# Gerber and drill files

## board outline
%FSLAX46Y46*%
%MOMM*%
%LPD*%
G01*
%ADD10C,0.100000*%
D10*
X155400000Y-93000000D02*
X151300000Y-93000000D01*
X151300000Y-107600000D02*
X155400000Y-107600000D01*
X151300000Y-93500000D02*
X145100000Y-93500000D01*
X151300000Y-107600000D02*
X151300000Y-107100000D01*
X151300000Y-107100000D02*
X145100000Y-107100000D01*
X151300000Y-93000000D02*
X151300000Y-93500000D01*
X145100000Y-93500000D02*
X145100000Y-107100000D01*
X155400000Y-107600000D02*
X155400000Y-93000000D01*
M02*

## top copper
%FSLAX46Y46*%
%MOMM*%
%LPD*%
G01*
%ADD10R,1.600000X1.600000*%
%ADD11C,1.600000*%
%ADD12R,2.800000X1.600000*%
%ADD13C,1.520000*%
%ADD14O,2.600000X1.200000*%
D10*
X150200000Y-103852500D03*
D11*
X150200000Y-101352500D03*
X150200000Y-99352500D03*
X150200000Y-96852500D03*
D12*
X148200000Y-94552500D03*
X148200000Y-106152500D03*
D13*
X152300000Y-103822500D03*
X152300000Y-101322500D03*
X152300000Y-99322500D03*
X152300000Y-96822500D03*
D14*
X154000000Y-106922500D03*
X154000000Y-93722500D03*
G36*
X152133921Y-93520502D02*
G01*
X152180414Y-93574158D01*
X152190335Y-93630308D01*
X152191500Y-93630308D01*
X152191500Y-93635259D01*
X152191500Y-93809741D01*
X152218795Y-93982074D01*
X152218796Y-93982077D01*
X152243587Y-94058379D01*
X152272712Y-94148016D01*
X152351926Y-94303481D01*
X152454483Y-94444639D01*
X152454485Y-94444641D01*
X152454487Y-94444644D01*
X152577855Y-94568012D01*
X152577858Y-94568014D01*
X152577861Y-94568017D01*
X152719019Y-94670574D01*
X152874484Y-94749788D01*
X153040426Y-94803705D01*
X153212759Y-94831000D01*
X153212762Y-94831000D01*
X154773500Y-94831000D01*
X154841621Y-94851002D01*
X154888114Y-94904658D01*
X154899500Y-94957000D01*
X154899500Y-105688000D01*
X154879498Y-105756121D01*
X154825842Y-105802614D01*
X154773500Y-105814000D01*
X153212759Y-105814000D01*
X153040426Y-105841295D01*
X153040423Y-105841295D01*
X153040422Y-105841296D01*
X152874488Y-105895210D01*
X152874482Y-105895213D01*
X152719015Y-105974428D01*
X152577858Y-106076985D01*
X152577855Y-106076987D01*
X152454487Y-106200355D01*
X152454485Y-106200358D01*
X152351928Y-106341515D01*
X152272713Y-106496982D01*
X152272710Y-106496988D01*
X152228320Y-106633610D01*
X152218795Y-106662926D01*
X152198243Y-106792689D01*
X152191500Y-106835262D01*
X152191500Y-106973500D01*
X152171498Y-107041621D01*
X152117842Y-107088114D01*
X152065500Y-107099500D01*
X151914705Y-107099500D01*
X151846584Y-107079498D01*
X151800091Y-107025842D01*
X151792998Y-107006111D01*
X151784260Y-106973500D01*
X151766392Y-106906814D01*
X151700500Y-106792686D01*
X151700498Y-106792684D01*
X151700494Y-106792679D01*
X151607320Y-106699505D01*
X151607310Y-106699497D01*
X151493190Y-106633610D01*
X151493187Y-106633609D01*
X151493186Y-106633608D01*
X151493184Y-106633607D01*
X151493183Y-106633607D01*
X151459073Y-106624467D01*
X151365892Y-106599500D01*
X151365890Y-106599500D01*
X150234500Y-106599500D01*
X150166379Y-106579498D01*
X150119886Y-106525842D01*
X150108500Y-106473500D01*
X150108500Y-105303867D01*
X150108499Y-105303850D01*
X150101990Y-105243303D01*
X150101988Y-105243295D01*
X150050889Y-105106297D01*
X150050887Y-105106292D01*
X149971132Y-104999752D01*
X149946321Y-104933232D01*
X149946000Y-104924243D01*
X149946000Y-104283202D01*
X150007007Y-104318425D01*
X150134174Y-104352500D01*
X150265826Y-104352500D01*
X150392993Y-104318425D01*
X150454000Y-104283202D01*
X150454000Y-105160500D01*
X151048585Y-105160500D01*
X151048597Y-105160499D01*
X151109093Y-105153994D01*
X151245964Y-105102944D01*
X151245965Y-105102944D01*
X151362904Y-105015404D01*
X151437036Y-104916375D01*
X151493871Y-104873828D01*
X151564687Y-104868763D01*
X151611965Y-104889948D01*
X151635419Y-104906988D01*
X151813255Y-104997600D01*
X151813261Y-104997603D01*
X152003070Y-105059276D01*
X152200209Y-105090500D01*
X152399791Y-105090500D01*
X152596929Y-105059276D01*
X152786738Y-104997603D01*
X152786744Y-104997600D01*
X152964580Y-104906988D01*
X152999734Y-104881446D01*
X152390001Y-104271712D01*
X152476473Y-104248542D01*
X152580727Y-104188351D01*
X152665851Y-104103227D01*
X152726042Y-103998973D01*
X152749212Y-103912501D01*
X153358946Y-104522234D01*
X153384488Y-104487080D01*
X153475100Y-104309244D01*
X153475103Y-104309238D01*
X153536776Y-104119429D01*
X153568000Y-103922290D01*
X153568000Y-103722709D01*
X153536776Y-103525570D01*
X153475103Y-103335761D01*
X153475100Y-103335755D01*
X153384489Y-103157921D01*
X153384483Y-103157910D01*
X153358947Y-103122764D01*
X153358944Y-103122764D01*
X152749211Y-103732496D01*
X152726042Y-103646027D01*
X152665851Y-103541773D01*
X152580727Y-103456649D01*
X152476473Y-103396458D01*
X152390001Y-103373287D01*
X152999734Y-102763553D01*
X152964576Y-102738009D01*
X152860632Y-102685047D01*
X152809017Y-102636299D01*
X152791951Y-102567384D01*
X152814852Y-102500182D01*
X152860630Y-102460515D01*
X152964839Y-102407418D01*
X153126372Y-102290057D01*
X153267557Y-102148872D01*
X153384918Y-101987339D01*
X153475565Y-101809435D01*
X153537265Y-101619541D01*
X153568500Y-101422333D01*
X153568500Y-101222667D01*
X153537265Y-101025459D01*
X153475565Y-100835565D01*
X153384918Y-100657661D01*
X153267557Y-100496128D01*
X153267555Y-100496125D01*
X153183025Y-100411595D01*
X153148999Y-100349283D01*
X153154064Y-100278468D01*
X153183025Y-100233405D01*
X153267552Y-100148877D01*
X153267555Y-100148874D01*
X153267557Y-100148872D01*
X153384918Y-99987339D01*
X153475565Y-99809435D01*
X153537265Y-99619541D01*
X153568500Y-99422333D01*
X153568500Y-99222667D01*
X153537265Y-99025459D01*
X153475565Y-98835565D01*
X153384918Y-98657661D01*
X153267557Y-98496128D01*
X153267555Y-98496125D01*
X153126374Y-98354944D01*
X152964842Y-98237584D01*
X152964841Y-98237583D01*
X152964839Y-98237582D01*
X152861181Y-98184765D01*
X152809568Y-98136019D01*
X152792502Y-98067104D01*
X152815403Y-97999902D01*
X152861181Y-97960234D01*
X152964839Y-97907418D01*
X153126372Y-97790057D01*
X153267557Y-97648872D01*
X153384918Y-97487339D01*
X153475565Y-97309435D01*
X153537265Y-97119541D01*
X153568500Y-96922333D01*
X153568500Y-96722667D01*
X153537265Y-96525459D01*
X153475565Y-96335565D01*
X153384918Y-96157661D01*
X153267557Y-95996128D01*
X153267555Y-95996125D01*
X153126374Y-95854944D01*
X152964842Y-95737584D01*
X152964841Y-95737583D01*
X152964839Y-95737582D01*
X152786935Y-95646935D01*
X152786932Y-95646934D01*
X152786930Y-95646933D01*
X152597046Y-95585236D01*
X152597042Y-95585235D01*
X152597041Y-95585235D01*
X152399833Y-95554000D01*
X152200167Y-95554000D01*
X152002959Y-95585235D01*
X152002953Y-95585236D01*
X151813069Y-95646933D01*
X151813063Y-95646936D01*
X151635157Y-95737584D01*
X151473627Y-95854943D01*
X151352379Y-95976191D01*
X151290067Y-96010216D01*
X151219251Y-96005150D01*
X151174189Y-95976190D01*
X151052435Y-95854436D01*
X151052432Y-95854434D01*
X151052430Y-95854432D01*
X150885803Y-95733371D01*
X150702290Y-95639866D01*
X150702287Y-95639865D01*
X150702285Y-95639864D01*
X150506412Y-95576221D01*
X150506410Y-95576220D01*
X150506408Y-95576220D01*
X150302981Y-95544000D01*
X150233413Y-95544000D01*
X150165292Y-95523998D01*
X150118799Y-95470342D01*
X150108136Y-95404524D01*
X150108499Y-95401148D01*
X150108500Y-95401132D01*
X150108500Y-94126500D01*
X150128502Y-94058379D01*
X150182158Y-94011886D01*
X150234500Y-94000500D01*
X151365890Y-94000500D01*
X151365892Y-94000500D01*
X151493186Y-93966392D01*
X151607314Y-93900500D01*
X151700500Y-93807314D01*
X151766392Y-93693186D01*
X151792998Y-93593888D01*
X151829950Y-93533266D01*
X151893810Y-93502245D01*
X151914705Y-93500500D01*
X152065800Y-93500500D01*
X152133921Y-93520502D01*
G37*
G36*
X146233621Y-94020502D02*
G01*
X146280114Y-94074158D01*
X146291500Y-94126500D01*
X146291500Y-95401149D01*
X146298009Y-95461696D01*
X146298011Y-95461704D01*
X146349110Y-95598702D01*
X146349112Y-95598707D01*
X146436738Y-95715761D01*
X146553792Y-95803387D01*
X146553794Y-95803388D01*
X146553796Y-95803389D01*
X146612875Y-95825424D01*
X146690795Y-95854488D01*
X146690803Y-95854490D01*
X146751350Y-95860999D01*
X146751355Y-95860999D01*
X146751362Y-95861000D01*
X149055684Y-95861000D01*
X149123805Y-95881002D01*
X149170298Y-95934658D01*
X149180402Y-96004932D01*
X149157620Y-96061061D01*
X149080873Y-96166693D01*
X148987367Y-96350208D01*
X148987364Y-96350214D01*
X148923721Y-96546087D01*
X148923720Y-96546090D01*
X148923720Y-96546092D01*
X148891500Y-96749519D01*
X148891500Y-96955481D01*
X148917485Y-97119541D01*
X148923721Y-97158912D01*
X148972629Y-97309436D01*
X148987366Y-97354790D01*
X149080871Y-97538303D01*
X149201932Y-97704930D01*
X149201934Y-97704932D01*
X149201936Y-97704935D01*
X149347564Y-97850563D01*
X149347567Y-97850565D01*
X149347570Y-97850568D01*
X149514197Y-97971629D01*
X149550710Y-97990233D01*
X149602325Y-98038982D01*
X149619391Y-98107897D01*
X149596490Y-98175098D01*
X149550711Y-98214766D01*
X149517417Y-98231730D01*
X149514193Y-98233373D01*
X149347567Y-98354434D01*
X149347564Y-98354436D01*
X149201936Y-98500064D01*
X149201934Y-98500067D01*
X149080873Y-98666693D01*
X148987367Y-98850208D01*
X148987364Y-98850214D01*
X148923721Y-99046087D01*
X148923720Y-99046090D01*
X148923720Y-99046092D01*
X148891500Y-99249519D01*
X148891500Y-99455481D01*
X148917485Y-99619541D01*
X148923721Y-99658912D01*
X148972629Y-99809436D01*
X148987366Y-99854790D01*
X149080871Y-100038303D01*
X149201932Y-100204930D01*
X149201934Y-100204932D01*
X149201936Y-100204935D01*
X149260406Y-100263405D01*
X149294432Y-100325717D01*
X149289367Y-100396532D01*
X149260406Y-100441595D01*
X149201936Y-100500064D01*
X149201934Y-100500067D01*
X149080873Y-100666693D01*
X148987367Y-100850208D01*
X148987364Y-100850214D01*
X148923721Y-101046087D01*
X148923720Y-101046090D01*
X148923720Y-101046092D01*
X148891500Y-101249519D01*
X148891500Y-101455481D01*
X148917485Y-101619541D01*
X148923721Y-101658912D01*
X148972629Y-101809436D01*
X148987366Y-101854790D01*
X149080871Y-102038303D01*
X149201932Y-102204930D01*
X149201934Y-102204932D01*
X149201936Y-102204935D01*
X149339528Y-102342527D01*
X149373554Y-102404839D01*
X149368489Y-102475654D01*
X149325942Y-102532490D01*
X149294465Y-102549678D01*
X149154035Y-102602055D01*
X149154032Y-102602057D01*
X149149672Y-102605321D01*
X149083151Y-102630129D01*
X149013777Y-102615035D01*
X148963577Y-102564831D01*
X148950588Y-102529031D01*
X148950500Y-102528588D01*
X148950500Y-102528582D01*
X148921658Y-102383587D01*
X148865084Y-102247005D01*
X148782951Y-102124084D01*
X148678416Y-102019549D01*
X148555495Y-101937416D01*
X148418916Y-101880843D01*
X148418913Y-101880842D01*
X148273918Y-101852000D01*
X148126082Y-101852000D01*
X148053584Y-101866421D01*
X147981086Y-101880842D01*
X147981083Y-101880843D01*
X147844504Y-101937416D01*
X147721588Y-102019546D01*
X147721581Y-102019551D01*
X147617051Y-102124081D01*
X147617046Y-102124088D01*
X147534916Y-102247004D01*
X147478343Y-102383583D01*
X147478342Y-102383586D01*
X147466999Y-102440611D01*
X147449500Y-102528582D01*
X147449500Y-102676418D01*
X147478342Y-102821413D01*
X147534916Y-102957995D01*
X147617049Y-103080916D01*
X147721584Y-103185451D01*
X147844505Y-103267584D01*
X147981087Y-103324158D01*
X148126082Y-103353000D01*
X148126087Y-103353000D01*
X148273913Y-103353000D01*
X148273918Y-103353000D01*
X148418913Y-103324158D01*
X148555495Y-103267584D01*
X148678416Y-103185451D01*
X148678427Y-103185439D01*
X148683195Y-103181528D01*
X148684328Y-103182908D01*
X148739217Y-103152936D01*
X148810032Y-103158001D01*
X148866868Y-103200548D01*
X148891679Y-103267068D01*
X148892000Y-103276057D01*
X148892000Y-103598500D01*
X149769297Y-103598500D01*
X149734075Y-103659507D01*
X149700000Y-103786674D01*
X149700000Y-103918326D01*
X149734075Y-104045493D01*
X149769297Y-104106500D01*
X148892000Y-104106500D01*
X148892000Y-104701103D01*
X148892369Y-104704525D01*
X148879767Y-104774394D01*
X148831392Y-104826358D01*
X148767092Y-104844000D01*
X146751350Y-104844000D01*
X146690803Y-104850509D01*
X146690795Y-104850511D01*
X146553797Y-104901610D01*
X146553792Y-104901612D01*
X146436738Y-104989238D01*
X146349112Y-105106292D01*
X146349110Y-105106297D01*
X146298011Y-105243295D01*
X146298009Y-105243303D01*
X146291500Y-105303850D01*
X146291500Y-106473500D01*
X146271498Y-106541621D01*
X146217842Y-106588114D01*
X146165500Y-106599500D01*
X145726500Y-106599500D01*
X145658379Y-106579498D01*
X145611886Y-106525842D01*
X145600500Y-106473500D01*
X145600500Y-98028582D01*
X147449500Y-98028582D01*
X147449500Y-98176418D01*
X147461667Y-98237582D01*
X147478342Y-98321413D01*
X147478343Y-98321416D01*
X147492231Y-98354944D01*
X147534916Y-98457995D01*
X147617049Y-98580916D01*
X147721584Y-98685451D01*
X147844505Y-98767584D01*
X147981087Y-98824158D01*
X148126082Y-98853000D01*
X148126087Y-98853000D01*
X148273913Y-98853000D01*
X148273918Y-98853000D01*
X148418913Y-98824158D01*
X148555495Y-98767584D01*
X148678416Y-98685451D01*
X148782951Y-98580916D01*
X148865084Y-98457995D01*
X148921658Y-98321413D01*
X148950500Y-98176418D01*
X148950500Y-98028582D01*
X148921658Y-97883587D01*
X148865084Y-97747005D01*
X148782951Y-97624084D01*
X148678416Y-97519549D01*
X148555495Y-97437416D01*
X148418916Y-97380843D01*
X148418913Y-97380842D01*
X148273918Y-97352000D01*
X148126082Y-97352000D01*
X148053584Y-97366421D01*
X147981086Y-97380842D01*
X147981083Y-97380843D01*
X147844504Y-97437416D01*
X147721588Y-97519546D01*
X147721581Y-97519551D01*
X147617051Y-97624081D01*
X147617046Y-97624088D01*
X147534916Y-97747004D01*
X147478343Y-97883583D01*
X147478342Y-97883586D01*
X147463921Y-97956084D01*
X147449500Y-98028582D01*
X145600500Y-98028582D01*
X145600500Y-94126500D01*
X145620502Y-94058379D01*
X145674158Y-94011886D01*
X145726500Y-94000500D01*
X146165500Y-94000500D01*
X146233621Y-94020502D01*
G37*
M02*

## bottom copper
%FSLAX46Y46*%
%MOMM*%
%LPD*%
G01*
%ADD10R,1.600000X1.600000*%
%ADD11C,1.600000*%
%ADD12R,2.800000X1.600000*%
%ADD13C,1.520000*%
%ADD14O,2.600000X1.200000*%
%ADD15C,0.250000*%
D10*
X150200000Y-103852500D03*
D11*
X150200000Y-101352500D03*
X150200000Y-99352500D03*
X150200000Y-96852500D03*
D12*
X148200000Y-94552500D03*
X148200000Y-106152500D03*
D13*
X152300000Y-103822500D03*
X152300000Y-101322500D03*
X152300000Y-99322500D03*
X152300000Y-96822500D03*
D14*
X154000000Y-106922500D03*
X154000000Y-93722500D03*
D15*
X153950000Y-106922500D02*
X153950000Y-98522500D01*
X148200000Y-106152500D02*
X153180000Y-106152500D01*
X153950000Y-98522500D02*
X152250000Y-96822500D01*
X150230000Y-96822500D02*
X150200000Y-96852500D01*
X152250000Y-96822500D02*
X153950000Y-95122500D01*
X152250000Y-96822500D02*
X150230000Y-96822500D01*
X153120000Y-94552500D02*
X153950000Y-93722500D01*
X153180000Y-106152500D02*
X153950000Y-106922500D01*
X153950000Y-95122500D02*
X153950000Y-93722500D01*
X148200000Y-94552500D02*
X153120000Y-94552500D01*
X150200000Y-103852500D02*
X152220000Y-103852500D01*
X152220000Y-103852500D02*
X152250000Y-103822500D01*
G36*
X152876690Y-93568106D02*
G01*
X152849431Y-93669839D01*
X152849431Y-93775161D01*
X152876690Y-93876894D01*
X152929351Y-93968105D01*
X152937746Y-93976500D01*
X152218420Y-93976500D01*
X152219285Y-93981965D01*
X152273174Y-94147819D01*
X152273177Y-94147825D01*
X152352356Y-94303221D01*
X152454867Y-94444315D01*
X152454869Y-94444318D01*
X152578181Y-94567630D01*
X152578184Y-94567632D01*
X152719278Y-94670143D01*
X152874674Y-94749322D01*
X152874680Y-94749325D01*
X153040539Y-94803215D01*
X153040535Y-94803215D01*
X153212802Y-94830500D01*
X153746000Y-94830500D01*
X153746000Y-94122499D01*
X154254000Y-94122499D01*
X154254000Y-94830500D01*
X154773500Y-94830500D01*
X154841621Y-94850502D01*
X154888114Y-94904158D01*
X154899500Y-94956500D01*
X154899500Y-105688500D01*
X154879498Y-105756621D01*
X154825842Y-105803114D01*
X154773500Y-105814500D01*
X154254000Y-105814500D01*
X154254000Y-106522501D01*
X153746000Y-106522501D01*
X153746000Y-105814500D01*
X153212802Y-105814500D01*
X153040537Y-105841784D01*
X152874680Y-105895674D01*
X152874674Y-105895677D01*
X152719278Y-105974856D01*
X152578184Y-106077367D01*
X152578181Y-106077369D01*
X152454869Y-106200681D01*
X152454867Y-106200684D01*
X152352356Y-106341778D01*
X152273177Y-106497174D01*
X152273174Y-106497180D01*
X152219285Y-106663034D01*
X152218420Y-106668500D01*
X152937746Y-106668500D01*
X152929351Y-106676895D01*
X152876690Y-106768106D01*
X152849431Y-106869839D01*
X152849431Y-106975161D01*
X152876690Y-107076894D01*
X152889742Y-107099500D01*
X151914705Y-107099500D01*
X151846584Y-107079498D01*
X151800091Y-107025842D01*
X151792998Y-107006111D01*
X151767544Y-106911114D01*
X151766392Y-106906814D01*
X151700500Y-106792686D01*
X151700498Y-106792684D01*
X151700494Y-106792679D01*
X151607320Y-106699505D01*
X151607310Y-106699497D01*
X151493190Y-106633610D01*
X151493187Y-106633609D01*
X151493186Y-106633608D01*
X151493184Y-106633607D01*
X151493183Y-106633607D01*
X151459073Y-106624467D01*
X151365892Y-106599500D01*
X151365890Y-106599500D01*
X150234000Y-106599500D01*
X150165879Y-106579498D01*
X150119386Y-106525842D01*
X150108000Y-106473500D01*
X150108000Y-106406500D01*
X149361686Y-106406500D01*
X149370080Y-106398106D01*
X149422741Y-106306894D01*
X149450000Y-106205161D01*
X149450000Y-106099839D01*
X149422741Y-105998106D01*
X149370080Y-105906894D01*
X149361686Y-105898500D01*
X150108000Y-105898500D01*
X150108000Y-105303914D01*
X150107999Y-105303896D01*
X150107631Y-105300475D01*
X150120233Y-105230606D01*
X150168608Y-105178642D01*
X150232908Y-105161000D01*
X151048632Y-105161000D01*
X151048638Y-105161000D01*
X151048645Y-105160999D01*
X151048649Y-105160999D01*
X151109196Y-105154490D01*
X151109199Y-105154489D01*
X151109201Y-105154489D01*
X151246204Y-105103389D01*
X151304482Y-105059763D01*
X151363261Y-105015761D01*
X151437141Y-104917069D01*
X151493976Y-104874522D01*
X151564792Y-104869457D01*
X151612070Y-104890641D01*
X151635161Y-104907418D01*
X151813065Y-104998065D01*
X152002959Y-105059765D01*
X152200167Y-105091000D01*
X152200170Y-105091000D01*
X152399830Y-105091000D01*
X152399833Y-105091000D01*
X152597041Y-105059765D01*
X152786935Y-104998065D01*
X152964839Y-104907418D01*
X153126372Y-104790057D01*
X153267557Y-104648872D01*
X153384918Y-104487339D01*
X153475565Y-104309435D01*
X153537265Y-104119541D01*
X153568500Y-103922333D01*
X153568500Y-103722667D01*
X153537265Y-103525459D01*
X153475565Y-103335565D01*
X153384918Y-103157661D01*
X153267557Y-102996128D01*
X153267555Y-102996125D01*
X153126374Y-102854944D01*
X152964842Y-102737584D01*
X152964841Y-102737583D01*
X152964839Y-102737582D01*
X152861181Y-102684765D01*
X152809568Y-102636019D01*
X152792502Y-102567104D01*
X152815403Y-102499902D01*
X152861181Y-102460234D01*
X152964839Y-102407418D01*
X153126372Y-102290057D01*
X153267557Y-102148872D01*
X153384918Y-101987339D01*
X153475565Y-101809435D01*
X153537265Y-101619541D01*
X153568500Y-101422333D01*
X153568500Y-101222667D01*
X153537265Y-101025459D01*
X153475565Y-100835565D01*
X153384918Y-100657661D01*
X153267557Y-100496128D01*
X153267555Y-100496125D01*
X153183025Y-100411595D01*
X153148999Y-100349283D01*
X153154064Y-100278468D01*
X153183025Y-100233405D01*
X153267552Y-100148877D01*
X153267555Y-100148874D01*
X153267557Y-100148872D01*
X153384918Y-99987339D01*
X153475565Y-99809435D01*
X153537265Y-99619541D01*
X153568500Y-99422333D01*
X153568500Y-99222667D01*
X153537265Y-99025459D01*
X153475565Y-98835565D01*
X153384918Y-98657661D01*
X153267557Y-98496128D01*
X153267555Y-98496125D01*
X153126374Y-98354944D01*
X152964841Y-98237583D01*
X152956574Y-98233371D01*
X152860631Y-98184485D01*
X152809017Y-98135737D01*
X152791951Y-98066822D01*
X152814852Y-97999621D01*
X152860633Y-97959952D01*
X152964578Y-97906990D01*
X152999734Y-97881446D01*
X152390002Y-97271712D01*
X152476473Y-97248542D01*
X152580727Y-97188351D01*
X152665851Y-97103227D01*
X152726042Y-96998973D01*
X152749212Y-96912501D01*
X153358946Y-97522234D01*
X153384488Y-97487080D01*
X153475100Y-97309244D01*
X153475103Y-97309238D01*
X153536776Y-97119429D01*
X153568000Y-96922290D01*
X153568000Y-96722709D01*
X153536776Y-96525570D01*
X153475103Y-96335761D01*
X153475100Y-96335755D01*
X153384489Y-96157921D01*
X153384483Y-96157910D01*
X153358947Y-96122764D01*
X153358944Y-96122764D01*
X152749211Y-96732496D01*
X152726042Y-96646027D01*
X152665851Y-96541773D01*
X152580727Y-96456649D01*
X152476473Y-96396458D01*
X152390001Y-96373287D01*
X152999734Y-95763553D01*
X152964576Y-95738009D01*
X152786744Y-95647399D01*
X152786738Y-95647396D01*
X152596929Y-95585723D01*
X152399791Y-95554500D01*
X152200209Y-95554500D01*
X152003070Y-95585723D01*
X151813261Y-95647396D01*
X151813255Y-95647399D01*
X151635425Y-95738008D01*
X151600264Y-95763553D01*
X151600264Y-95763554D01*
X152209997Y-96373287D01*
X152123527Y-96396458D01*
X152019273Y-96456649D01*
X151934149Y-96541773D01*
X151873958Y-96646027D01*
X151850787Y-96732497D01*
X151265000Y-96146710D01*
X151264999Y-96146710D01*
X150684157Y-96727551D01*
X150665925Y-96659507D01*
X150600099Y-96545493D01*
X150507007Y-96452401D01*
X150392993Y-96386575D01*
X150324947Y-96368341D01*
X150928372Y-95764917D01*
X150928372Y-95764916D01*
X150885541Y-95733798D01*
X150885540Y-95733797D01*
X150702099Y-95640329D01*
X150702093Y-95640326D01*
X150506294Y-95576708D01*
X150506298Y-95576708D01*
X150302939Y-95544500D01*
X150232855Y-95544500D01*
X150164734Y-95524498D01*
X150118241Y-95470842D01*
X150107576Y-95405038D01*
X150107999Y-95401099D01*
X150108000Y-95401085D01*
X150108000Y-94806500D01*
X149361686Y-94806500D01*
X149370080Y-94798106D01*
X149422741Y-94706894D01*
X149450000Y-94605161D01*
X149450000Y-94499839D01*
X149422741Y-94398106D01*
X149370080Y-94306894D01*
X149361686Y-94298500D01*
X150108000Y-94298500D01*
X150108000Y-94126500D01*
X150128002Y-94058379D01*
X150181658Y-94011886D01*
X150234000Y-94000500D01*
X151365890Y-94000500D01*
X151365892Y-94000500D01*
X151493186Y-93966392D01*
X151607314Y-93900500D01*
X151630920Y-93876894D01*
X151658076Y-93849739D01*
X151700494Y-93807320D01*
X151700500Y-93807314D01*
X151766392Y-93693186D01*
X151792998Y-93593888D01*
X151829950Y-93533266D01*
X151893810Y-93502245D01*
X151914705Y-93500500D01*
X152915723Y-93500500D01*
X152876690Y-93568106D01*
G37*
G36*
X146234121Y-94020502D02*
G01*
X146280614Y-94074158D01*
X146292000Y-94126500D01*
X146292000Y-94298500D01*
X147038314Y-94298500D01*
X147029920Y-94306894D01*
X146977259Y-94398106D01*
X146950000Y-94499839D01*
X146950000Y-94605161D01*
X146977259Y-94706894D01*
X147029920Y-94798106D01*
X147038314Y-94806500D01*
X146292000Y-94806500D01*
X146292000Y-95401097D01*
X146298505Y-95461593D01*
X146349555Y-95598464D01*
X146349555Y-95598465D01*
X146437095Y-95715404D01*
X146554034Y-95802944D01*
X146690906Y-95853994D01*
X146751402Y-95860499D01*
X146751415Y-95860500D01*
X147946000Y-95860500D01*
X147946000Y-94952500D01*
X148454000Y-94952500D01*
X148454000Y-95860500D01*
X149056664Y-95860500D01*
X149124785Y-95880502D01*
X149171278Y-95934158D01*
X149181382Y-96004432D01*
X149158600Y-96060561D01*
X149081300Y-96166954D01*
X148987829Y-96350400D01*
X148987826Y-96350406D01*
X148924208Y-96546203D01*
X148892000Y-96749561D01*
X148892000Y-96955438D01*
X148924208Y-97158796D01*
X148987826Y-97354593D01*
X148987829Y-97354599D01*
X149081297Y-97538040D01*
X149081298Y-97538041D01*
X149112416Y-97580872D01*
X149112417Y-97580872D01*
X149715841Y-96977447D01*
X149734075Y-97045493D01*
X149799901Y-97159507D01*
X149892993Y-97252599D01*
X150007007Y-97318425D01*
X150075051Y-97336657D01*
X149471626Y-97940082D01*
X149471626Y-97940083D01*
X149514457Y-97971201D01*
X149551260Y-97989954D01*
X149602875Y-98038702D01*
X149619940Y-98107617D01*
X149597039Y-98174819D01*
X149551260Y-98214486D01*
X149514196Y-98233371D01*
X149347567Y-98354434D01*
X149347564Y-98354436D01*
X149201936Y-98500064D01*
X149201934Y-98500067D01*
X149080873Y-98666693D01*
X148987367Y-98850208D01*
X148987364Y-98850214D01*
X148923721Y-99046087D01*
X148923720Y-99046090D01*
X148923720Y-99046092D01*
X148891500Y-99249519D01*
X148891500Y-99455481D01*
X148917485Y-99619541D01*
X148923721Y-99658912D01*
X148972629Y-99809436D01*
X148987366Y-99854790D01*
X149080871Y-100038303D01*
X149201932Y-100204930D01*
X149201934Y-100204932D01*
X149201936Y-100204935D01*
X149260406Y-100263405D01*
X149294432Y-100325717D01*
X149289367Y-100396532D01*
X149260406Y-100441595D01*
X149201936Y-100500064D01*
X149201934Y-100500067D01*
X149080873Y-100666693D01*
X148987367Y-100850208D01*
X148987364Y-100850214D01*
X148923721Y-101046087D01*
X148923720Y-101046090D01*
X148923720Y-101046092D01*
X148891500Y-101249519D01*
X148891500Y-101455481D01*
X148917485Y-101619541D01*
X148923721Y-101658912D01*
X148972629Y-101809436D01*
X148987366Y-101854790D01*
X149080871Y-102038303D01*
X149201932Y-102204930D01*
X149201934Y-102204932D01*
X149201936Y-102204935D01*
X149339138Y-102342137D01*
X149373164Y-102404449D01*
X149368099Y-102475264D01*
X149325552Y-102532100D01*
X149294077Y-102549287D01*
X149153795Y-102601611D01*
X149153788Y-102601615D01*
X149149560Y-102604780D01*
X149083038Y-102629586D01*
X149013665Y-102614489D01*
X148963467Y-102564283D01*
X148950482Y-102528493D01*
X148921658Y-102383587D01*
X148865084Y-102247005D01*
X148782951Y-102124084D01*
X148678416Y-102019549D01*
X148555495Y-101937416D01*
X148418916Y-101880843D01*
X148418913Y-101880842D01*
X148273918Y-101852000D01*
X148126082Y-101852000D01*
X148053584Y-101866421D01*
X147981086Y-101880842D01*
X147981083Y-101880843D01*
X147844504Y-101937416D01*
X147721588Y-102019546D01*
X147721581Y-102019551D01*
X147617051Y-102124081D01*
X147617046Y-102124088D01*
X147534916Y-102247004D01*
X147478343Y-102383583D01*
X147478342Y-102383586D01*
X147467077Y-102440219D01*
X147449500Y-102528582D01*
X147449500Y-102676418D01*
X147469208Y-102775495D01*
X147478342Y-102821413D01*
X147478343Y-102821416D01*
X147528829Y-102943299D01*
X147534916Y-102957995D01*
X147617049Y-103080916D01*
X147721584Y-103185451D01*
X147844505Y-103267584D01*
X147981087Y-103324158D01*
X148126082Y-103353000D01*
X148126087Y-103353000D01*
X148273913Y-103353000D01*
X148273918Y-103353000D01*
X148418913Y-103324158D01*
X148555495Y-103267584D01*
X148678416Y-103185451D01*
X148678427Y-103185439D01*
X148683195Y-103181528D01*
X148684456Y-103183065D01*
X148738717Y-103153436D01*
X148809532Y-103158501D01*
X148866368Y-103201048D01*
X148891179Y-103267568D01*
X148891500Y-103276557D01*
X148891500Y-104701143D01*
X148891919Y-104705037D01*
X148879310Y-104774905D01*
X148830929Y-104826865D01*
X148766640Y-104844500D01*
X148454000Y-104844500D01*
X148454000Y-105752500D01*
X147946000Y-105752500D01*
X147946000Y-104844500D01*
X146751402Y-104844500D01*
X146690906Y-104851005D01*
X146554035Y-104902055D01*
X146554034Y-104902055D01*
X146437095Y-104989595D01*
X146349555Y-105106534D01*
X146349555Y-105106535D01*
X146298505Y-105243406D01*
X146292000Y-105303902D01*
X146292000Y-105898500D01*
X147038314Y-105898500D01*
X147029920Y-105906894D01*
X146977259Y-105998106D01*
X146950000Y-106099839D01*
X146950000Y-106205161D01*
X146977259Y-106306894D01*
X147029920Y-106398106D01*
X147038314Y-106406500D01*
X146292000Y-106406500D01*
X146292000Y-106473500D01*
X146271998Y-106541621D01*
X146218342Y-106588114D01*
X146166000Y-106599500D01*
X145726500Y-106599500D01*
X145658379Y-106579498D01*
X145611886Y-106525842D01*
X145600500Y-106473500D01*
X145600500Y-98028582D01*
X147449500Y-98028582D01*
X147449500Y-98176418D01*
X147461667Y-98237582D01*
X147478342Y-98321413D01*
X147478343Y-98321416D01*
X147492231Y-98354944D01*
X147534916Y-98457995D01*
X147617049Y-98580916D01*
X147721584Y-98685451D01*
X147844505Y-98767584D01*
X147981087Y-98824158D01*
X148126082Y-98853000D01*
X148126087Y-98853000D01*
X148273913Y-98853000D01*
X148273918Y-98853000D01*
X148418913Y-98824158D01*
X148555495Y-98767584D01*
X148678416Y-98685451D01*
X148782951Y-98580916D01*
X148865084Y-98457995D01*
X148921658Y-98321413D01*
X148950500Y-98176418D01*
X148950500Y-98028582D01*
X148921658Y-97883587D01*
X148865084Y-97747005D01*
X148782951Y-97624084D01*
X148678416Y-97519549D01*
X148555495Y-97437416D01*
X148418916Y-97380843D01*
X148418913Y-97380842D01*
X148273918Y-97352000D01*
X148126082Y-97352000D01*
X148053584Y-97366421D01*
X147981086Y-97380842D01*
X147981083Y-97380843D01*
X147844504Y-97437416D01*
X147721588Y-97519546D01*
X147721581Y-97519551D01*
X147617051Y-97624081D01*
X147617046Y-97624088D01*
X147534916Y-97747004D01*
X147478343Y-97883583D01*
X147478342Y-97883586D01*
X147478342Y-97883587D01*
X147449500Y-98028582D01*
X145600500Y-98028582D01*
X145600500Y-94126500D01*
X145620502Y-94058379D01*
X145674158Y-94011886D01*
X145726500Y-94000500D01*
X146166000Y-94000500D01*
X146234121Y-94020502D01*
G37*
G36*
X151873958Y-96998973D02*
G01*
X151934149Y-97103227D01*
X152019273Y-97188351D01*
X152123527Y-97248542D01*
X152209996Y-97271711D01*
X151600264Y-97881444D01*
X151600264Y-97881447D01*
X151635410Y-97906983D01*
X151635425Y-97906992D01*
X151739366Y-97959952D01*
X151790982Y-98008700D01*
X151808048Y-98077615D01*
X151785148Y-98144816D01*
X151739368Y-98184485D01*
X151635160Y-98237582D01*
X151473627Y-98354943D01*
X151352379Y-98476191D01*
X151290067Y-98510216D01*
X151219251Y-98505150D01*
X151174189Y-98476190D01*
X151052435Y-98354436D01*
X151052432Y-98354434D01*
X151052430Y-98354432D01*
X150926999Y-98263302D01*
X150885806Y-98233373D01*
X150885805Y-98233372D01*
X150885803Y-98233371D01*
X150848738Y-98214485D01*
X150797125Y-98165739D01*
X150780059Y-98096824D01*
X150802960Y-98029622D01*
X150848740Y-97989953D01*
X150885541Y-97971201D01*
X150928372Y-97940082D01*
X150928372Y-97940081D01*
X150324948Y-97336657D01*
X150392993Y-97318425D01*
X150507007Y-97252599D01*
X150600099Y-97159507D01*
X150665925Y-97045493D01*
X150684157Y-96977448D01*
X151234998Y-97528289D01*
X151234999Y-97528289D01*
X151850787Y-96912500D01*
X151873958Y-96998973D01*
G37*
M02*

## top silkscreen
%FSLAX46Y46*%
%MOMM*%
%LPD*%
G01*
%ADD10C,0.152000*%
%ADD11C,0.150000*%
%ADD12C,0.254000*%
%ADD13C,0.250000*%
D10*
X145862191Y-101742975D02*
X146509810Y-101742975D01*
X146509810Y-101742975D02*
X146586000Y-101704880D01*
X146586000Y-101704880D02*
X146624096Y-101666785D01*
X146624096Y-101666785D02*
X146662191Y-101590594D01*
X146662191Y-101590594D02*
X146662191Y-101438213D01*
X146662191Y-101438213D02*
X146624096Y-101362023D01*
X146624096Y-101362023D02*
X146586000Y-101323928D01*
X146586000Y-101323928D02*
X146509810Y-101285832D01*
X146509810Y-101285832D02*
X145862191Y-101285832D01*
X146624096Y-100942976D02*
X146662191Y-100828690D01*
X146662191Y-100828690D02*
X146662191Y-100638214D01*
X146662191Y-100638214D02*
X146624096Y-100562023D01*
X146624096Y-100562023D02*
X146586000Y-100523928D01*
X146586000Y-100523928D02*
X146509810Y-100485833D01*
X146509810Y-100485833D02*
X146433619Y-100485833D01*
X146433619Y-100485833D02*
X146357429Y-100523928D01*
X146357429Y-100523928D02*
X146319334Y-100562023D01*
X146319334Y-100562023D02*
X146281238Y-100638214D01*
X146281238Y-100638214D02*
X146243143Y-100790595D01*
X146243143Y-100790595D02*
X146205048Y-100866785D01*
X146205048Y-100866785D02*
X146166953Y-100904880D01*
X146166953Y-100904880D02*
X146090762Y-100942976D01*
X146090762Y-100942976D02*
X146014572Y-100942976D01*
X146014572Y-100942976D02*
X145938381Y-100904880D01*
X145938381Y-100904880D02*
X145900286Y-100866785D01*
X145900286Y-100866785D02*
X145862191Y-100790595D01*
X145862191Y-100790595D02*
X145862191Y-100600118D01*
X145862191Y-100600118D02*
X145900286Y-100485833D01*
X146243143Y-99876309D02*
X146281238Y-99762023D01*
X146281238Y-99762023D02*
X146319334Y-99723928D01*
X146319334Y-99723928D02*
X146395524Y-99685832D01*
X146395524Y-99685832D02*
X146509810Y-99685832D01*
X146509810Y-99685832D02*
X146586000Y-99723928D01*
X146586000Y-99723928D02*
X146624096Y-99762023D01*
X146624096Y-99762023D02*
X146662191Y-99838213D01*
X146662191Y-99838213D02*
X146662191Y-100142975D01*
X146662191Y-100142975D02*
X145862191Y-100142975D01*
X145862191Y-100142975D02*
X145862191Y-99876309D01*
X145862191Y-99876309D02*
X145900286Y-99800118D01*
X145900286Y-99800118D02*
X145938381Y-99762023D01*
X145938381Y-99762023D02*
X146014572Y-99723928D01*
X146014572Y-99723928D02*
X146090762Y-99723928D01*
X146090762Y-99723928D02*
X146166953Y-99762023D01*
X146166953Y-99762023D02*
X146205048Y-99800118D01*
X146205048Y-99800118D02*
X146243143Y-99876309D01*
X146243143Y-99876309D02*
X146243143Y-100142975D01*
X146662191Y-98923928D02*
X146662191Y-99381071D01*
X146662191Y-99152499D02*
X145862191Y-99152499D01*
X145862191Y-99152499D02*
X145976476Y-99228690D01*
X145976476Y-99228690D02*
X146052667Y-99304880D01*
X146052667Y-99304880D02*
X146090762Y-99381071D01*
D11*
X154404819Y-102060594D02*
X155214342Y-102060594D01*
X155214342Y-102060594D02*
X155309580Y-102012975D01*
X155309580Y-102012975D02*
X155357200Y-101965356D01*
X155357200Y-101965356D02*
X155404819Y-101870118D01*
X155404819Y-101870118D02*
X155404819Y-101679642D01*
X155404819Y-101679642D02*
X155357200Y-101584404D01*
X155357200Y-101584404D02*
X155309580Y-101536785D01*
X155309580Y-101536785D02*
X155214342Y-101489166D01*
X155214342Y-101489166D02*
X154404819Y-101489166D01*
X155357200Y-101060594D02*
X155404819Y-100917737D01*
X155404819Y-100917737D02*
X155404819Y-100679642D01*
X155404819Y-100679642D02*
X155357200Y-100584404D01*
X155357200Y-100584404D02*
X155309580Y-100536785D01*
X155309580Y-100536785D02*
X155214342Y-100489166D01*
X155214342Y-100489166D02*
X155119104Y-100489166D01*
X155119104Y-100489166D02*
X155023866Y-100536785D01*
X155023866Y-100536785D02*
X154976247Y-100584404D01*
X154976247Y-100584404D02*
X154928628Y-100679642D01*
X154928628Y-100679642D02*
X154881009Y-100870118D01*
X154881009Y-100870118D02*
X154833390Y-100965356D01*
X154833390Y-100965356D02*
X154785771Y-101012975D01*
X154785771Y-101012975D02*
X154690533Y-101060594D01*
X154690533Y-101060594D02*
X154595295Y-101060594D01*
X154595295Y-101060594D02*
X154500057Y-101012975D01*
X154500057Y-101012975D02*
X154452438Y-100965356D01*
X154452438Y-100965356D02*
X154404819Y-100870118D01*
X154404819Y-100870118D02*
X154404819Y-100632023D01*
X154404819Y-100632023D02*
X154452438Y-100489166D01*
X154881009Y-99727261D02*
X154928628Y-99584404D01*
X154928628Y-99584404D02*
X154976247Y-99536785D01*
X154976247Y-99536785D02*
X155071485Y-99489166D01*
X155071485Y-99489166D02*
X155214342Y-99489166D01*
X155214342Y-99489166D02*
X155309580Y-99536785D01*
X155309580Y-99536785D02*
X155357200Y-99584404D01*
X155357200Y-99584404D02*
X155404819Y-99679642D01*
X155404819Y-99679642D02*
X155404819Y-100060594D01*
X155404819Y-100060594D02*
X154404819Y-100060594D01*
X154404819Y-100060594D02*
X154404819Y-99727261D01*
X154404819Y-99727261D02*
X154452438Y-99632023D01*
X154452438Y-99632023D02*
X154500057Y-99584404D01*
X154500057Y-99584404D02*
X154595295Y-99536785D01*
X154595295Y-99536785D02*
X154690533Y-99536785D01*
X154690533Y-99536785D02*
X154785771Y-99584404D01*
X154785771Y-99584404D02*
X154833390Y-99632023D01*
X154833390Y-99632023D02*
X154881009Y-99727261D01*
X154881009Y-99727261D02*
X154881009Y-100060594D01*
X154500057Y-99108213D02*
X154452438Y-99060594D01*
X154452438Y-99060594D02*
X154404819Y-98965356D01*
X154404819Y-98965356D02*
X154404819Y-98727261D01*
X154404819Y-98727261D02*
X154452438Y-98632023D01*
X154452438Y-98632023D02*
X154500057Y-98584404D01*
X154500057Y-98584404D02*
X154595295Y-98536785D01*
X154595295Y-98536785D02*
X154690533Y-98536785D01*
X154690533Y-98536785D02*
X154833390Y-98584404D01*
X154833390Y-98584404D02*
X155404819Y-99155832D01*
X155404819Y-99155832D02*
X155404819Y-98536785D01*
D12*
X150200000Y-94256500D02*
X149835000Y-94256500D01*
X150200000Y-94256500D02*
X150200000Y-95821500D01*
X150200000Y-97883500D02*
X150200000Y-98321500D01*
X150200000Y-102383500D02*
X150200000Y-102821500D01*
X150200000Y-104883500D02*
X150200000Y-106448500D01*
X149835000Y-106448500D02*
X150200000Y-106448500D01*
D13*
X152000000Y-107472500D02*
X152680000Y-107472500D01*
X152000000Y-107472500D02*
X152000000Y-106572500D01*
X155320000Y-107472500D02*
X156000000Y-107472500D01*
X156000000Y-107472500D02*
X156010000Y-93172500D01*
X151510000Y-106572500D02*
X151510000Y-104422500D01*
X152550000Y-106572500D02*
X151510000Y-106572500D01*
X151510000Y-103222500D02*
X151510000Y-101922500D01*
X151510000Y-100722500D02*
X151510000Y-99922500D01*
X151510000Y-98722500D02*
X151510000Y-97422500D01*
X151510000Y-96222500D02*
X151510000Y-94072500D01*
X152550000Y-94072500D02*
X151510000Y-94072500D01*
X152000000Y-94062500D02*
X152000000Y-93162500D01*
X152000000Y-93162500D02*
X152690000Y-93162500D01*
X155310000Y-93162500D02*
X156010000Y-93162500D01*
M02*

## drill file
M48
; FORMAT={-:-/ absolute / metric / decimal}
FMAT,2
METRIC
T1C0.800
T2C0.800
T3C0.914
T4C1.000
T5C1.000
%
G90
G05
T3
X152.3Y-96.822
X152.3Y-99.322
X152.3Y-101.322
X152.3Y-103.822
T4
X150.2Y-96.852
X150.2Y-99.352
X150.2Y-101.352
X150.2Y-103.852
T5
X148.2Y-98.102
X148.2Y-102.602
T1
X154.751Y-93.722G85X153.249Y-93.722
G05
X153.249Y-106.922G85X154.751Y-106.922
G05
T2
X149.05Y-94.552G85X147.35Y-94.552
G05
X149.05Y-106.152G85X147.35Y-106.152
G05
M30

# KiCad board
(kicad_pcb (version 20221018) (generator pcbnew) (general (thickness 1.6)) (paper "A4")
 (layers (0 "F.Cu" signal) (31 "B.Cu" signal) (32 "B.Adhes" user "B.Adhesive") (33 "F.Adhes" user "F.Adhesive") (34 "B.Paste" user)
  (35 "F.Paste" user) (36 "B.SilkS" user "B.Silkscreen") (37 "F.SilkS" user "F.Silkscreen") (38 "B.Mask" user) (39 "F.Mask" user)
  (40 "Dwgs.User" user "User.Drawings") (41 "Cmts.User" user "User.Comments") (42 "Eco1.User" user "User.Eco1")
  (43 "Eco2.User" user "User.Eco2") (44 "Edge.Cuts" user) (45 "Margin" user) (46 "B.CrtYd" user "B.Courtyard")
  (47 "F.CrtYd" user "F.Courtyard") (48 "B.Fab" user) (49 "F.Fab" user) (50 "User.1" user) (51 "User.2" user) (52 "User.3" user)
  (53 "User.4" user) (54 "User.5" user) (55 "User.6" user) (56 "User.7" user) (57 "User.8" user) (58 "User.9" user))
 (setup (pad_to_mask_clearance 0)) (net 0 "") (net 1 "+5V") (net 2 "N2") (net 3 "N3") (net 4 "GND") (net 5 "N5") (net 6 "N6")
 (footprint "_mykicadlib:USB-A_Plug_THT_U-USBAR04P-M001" (layer "F.Cu") (at 149 100.3525 -90)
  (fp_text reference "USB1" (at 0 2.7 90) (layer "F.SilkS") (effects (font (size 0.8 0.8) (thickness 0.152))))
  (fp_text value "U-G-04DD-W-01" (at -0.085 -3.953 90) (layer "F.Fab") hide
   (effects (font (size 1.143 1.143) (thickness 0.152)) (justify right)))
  (fp_line (start -6.096 -1.2) (end -6.096 -0.835) (stroke (width 0.254) (type solid)) (layer "F.SilkS"))
  (fp_line (start -6.096 -1.2) (end -4.531 -1.2) (stroke (width 0.254) (type solid)) (layer "F.SilkS"))
  (fp_line (start -2.469 -1.2) (end -2.031 -1.2) (stroke (width 0.254) (type solid)) (layer "F.SilkS"))
  (fp_line (start 2.031 -1.2) (end 2.469 -1.2) (stroke (width 0.254) (type solid)) (layer "F.SilkS"))
  (fp_line (start 4.531 -1.2) (end 6.096 -1.2) (stroke (width 0.254) (type solid)) (layer "F.SilkS"))
  (fp_line (start 6.096 -0.835) (end 6.096 -1.2) (stroke (width 0.254) (type solid)) (layer "F.SilkS"))
  (pad "" np_thru_hole circle (at -2.25 0.8 270) (size 1 1) (drill 1) (layers "*.Cu" "*.Mask"))
  (pad "" np_thru_hole circle (at 2.25 0.8 270) (size 1 1) (drill 1) (layers "*.Cu" "*.Mask"))
  (pad "1" thru_hole rect (at 3.5 -1.2 270) (size 1.6 1.6) (drill 1) (layers "*.Cu" "*.Mask") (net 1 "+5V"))
  (pad "2" thru_hole circle (at 1 -1.2 270) (size 1.6 1.6) (drill 1) (layers "*.Cu" "*.Mask") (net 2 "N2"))
  (pad "3" thru_hole circle (at -1 -1.2 270) (size 1.6 1.6) (drill 1) (layers "*.Cu" "*.Mask") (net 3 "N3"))
  (pad "4" thru_hole circle (at -3.5 -1.2 270) (size 1.6 1.6) (drill 1) (layers "*.Cu" "*.Mask") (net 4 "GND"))
  (pad "5" thru_hole rect (at -5.8 0.8 270) (size 1.6 2.8) (drill oval 0.8 2.5) (layers "*.Cu" "*.Mask") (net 4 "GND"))
  (pad "5" thru_hole rect (at 5.8 0.8 270) (size 1.6 2.8) (drill oval 0.8 2.5) (layers "*.Cu" "*.Mask") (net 4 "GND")))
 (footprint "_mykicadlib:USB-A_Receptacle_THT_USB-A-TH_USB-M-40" (layer "F.Cu") (at 153.41 100.3225 90)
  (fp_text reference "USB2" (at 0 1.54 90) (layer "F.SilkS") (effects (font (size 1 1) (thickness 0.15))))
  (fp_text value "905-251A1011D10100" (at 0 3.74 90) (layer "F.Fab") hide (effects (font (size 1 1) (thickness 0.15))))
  (fp_line (start -7.15 -1.41) (end -7.15 -0.73) (stroke (width 0.25) (type solid)) (layer "F.SilkS"))
  (fp_line (start -7.15 -1.41) (end -6.25 -1.41) (stroke (width 0.25) (type solid)) (layer "F.SilkS"))
  (fp_line (start -7.15 1.91) (end -7.15 2.59) (stroke (width 0.25) (type solid)) (layer "F.SilkS"))
  (fp_line (start -7.15 2.59) (end 7.15 2.6) (stroke (width 0.25) (type solid)) (layer "F.SilkS"))
  (fp_line (start -6.25 -1.9) (end -4.1 -1.9) (stroke (width 0.25) (type solid)) (layer "F.SilkS"))
  (fp_line (start -6.25 -0.86) (end -6.25 -1.9) (stroke (width 0.25) (type solid)) (layer "F.SilkS"))
  (fp_line (start -2.9 -1.9) (end -1.6 -1.9) (stroke (width 0.25) (type solid)) (layer "F.SilkS"))
  (fp_line (start -0.4 -1.9) (end 0.4 -1.9) (stroke (width 0.25) (type solid)) (layer "F.SilkS"))
  (fp_line (start 1.6 -1.9) (end 2.9 -1.9) (stroke (width 0.25) (type solid)) (layer "F.SilkS"))
  (fp_line (start 4.1 -1.9) (end 6.25 -1.9) (stroke (width 0.25) (type solid)) (layer "F.SilkS"))
  (fp_line (start 6.25 -0.86) (end 6.25 -1.9) (stroke (width 0.25) (type solid)) (layer "F.SilkS"))
  (fp_line (start 6.26 -1.41) (end 7.16 -1.41) (stroke (width 0.25) (type solid)) (layer "F.SilkS"))
  (fp_line (start 7.16 -1.41) (end 7.16 -0.72) (stroke (width 0.25) (type solid)) (layer "F.SilkS"))
  (fp_line (start 7.16 1.9) (end 7.16 2.6) (stroke (width 0.25) (type solid)) (layer "F.SilkS"))
  (pad "1" thru_hole circle (at -3.5 -1.11 90) (size 1.52 1.52) (drill 0.9144) (layers "*.Cu" "*.Paste" "*.Mask") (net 1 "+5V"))
  (pad "2" thru_hole circle (at -1 -1.11 90) (size 1.52 1.52) (drill 0.9144) (layers "*.Cu" "*.Paste" "*.Mask") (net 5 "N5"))
  (pad "3" thru_hole circle (at 1 -1.11 90) (size 1.52 1.52) (drill 0.9144) (layers "*.Cu" "*.Paste" "*.Mask") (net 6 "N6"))
  (pad "4" thru_hole circle (at 3.5 -1.11 90) (size 1.52 1.52) (drill 0.9144) (layers "*.Cu" "*.Paste" "*.Mask") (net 4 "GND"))
  (pad "5" thru_hole oval (at -6.6 0.59) (size 2.6 1.2) (drill oval 2.301138 0.799998) (layers "*.Cu" "*.Paste" "*.Mask") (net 4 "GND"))
  (pad "5" thru_hole oval (at 6.6 0.59 180) (size 2.6 1.2) (drill oval 2.301138 0.799998) (layers "*.Cu" "*.Paste" "*.Mask") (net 4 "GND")))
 (gr_line (start 155.4 93) (end 151.3 93) (stroke (width 0.1) (type solid)) (layer "Edge.Cuts"))
 (gr_line (start 151.3 107.6) (end 155.4 107.6) (stroke (width 0.1) (type solid)) (layer "Edge.Cuts"))
 (gr_line (start 151.3 93.5) (end 145.1 93.5) (stroke (width 0.1) (type solid)) (layer "Edge.Cuts"))
 (gr_line (start 151.3 107.6) (end 151.3 107.1) (stroke (width 0.1) (type solid)) (layer "Edge.Cuts"))
 (gr_line (start 151.3 107.1) (end 145.1 107.1) (stroke (width 0.1) (type solid)) (layer "Edge.Cuts"))
 (gr_line (start 151.3 93) (end 151.3 93.5) (stroke (width 0.1) (type solid)) (layer "Edge.Cuts"))
 (gr_line (start 145.1 93.5) (end 145.1 107.1) (stroke (width 0.1) (type solid)) (layer "Edge.Cuts"))
 (gr_line (start 155.4 107.6) (end 155.4 93) (stroke (width 0.1) (type solid)) (layer "Edge.Cuts"))
 (segment (start 153.95 106.9225) (end 153.95 98.5225) (width 0.25) (layer "B.Cu") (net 4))
 (segment (start 148.2 106.1525) (end 153.18 106.1525) (width 0.25) (layer "B.Cu") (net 4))
 (segment (start 153.95 98.5225) (end 152.25 96.8225) (width 0.25) (layer "B.Cu") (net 4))
 (segment (start 150.23 96.8225) (end 150.2 96.8525) (width 0.25) (layer "B.Cu") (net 4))
 (segment (start 152.25 96.8225) (end 153.95 95.1225) (width 0.25) (layer "B.Cu") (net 4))
 (segment (start 152.25 96.8225) (end 150.23 96.8225) (width 0.25) (layer "B.Cu") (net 4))
 (segment (start 153.12 94.5525) (end 153.95 93.7225) (width 0.25) (layer "B.Cu") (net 4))
 (segment (start 153.18 106.1525) (end 153.95 106.9225) (width 0.25) (layer "B.Cu") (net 4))
 (segment (start 153.95 95.1225) (end 153.95 93.7225) (width 0.25) (layer "B.Cu") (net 4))
 (segment (start 148.2 94.5525) (end 153.12 94.5525) (width 0.25) (layer "B.Cu") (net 4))
 (segment (start 150.2 103.8525) (end 152.22 103.8525) (width 0.25) (layer "B.Cu") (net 1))
 (segment (start 152.22 103.8525) (end 152.25 103.8225) (width 0.25) (layer "B.Cu") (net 1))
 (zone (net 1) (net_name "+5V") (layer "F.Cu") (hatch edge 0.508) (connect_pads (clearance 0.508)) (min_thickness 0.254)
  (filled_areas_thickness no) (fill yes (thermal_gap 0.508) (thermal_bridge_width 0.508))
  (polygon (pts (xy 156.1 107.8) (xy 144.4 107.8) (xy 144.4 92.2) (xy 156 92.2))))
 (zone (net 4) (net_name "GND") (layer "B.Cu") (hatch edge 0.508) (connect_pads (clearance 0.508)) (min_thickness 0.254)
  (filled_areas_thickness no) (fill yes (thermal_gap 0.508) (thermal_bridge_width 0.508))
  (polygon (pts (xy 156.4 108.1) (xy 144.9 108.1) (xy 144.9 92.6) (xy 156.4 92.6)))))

